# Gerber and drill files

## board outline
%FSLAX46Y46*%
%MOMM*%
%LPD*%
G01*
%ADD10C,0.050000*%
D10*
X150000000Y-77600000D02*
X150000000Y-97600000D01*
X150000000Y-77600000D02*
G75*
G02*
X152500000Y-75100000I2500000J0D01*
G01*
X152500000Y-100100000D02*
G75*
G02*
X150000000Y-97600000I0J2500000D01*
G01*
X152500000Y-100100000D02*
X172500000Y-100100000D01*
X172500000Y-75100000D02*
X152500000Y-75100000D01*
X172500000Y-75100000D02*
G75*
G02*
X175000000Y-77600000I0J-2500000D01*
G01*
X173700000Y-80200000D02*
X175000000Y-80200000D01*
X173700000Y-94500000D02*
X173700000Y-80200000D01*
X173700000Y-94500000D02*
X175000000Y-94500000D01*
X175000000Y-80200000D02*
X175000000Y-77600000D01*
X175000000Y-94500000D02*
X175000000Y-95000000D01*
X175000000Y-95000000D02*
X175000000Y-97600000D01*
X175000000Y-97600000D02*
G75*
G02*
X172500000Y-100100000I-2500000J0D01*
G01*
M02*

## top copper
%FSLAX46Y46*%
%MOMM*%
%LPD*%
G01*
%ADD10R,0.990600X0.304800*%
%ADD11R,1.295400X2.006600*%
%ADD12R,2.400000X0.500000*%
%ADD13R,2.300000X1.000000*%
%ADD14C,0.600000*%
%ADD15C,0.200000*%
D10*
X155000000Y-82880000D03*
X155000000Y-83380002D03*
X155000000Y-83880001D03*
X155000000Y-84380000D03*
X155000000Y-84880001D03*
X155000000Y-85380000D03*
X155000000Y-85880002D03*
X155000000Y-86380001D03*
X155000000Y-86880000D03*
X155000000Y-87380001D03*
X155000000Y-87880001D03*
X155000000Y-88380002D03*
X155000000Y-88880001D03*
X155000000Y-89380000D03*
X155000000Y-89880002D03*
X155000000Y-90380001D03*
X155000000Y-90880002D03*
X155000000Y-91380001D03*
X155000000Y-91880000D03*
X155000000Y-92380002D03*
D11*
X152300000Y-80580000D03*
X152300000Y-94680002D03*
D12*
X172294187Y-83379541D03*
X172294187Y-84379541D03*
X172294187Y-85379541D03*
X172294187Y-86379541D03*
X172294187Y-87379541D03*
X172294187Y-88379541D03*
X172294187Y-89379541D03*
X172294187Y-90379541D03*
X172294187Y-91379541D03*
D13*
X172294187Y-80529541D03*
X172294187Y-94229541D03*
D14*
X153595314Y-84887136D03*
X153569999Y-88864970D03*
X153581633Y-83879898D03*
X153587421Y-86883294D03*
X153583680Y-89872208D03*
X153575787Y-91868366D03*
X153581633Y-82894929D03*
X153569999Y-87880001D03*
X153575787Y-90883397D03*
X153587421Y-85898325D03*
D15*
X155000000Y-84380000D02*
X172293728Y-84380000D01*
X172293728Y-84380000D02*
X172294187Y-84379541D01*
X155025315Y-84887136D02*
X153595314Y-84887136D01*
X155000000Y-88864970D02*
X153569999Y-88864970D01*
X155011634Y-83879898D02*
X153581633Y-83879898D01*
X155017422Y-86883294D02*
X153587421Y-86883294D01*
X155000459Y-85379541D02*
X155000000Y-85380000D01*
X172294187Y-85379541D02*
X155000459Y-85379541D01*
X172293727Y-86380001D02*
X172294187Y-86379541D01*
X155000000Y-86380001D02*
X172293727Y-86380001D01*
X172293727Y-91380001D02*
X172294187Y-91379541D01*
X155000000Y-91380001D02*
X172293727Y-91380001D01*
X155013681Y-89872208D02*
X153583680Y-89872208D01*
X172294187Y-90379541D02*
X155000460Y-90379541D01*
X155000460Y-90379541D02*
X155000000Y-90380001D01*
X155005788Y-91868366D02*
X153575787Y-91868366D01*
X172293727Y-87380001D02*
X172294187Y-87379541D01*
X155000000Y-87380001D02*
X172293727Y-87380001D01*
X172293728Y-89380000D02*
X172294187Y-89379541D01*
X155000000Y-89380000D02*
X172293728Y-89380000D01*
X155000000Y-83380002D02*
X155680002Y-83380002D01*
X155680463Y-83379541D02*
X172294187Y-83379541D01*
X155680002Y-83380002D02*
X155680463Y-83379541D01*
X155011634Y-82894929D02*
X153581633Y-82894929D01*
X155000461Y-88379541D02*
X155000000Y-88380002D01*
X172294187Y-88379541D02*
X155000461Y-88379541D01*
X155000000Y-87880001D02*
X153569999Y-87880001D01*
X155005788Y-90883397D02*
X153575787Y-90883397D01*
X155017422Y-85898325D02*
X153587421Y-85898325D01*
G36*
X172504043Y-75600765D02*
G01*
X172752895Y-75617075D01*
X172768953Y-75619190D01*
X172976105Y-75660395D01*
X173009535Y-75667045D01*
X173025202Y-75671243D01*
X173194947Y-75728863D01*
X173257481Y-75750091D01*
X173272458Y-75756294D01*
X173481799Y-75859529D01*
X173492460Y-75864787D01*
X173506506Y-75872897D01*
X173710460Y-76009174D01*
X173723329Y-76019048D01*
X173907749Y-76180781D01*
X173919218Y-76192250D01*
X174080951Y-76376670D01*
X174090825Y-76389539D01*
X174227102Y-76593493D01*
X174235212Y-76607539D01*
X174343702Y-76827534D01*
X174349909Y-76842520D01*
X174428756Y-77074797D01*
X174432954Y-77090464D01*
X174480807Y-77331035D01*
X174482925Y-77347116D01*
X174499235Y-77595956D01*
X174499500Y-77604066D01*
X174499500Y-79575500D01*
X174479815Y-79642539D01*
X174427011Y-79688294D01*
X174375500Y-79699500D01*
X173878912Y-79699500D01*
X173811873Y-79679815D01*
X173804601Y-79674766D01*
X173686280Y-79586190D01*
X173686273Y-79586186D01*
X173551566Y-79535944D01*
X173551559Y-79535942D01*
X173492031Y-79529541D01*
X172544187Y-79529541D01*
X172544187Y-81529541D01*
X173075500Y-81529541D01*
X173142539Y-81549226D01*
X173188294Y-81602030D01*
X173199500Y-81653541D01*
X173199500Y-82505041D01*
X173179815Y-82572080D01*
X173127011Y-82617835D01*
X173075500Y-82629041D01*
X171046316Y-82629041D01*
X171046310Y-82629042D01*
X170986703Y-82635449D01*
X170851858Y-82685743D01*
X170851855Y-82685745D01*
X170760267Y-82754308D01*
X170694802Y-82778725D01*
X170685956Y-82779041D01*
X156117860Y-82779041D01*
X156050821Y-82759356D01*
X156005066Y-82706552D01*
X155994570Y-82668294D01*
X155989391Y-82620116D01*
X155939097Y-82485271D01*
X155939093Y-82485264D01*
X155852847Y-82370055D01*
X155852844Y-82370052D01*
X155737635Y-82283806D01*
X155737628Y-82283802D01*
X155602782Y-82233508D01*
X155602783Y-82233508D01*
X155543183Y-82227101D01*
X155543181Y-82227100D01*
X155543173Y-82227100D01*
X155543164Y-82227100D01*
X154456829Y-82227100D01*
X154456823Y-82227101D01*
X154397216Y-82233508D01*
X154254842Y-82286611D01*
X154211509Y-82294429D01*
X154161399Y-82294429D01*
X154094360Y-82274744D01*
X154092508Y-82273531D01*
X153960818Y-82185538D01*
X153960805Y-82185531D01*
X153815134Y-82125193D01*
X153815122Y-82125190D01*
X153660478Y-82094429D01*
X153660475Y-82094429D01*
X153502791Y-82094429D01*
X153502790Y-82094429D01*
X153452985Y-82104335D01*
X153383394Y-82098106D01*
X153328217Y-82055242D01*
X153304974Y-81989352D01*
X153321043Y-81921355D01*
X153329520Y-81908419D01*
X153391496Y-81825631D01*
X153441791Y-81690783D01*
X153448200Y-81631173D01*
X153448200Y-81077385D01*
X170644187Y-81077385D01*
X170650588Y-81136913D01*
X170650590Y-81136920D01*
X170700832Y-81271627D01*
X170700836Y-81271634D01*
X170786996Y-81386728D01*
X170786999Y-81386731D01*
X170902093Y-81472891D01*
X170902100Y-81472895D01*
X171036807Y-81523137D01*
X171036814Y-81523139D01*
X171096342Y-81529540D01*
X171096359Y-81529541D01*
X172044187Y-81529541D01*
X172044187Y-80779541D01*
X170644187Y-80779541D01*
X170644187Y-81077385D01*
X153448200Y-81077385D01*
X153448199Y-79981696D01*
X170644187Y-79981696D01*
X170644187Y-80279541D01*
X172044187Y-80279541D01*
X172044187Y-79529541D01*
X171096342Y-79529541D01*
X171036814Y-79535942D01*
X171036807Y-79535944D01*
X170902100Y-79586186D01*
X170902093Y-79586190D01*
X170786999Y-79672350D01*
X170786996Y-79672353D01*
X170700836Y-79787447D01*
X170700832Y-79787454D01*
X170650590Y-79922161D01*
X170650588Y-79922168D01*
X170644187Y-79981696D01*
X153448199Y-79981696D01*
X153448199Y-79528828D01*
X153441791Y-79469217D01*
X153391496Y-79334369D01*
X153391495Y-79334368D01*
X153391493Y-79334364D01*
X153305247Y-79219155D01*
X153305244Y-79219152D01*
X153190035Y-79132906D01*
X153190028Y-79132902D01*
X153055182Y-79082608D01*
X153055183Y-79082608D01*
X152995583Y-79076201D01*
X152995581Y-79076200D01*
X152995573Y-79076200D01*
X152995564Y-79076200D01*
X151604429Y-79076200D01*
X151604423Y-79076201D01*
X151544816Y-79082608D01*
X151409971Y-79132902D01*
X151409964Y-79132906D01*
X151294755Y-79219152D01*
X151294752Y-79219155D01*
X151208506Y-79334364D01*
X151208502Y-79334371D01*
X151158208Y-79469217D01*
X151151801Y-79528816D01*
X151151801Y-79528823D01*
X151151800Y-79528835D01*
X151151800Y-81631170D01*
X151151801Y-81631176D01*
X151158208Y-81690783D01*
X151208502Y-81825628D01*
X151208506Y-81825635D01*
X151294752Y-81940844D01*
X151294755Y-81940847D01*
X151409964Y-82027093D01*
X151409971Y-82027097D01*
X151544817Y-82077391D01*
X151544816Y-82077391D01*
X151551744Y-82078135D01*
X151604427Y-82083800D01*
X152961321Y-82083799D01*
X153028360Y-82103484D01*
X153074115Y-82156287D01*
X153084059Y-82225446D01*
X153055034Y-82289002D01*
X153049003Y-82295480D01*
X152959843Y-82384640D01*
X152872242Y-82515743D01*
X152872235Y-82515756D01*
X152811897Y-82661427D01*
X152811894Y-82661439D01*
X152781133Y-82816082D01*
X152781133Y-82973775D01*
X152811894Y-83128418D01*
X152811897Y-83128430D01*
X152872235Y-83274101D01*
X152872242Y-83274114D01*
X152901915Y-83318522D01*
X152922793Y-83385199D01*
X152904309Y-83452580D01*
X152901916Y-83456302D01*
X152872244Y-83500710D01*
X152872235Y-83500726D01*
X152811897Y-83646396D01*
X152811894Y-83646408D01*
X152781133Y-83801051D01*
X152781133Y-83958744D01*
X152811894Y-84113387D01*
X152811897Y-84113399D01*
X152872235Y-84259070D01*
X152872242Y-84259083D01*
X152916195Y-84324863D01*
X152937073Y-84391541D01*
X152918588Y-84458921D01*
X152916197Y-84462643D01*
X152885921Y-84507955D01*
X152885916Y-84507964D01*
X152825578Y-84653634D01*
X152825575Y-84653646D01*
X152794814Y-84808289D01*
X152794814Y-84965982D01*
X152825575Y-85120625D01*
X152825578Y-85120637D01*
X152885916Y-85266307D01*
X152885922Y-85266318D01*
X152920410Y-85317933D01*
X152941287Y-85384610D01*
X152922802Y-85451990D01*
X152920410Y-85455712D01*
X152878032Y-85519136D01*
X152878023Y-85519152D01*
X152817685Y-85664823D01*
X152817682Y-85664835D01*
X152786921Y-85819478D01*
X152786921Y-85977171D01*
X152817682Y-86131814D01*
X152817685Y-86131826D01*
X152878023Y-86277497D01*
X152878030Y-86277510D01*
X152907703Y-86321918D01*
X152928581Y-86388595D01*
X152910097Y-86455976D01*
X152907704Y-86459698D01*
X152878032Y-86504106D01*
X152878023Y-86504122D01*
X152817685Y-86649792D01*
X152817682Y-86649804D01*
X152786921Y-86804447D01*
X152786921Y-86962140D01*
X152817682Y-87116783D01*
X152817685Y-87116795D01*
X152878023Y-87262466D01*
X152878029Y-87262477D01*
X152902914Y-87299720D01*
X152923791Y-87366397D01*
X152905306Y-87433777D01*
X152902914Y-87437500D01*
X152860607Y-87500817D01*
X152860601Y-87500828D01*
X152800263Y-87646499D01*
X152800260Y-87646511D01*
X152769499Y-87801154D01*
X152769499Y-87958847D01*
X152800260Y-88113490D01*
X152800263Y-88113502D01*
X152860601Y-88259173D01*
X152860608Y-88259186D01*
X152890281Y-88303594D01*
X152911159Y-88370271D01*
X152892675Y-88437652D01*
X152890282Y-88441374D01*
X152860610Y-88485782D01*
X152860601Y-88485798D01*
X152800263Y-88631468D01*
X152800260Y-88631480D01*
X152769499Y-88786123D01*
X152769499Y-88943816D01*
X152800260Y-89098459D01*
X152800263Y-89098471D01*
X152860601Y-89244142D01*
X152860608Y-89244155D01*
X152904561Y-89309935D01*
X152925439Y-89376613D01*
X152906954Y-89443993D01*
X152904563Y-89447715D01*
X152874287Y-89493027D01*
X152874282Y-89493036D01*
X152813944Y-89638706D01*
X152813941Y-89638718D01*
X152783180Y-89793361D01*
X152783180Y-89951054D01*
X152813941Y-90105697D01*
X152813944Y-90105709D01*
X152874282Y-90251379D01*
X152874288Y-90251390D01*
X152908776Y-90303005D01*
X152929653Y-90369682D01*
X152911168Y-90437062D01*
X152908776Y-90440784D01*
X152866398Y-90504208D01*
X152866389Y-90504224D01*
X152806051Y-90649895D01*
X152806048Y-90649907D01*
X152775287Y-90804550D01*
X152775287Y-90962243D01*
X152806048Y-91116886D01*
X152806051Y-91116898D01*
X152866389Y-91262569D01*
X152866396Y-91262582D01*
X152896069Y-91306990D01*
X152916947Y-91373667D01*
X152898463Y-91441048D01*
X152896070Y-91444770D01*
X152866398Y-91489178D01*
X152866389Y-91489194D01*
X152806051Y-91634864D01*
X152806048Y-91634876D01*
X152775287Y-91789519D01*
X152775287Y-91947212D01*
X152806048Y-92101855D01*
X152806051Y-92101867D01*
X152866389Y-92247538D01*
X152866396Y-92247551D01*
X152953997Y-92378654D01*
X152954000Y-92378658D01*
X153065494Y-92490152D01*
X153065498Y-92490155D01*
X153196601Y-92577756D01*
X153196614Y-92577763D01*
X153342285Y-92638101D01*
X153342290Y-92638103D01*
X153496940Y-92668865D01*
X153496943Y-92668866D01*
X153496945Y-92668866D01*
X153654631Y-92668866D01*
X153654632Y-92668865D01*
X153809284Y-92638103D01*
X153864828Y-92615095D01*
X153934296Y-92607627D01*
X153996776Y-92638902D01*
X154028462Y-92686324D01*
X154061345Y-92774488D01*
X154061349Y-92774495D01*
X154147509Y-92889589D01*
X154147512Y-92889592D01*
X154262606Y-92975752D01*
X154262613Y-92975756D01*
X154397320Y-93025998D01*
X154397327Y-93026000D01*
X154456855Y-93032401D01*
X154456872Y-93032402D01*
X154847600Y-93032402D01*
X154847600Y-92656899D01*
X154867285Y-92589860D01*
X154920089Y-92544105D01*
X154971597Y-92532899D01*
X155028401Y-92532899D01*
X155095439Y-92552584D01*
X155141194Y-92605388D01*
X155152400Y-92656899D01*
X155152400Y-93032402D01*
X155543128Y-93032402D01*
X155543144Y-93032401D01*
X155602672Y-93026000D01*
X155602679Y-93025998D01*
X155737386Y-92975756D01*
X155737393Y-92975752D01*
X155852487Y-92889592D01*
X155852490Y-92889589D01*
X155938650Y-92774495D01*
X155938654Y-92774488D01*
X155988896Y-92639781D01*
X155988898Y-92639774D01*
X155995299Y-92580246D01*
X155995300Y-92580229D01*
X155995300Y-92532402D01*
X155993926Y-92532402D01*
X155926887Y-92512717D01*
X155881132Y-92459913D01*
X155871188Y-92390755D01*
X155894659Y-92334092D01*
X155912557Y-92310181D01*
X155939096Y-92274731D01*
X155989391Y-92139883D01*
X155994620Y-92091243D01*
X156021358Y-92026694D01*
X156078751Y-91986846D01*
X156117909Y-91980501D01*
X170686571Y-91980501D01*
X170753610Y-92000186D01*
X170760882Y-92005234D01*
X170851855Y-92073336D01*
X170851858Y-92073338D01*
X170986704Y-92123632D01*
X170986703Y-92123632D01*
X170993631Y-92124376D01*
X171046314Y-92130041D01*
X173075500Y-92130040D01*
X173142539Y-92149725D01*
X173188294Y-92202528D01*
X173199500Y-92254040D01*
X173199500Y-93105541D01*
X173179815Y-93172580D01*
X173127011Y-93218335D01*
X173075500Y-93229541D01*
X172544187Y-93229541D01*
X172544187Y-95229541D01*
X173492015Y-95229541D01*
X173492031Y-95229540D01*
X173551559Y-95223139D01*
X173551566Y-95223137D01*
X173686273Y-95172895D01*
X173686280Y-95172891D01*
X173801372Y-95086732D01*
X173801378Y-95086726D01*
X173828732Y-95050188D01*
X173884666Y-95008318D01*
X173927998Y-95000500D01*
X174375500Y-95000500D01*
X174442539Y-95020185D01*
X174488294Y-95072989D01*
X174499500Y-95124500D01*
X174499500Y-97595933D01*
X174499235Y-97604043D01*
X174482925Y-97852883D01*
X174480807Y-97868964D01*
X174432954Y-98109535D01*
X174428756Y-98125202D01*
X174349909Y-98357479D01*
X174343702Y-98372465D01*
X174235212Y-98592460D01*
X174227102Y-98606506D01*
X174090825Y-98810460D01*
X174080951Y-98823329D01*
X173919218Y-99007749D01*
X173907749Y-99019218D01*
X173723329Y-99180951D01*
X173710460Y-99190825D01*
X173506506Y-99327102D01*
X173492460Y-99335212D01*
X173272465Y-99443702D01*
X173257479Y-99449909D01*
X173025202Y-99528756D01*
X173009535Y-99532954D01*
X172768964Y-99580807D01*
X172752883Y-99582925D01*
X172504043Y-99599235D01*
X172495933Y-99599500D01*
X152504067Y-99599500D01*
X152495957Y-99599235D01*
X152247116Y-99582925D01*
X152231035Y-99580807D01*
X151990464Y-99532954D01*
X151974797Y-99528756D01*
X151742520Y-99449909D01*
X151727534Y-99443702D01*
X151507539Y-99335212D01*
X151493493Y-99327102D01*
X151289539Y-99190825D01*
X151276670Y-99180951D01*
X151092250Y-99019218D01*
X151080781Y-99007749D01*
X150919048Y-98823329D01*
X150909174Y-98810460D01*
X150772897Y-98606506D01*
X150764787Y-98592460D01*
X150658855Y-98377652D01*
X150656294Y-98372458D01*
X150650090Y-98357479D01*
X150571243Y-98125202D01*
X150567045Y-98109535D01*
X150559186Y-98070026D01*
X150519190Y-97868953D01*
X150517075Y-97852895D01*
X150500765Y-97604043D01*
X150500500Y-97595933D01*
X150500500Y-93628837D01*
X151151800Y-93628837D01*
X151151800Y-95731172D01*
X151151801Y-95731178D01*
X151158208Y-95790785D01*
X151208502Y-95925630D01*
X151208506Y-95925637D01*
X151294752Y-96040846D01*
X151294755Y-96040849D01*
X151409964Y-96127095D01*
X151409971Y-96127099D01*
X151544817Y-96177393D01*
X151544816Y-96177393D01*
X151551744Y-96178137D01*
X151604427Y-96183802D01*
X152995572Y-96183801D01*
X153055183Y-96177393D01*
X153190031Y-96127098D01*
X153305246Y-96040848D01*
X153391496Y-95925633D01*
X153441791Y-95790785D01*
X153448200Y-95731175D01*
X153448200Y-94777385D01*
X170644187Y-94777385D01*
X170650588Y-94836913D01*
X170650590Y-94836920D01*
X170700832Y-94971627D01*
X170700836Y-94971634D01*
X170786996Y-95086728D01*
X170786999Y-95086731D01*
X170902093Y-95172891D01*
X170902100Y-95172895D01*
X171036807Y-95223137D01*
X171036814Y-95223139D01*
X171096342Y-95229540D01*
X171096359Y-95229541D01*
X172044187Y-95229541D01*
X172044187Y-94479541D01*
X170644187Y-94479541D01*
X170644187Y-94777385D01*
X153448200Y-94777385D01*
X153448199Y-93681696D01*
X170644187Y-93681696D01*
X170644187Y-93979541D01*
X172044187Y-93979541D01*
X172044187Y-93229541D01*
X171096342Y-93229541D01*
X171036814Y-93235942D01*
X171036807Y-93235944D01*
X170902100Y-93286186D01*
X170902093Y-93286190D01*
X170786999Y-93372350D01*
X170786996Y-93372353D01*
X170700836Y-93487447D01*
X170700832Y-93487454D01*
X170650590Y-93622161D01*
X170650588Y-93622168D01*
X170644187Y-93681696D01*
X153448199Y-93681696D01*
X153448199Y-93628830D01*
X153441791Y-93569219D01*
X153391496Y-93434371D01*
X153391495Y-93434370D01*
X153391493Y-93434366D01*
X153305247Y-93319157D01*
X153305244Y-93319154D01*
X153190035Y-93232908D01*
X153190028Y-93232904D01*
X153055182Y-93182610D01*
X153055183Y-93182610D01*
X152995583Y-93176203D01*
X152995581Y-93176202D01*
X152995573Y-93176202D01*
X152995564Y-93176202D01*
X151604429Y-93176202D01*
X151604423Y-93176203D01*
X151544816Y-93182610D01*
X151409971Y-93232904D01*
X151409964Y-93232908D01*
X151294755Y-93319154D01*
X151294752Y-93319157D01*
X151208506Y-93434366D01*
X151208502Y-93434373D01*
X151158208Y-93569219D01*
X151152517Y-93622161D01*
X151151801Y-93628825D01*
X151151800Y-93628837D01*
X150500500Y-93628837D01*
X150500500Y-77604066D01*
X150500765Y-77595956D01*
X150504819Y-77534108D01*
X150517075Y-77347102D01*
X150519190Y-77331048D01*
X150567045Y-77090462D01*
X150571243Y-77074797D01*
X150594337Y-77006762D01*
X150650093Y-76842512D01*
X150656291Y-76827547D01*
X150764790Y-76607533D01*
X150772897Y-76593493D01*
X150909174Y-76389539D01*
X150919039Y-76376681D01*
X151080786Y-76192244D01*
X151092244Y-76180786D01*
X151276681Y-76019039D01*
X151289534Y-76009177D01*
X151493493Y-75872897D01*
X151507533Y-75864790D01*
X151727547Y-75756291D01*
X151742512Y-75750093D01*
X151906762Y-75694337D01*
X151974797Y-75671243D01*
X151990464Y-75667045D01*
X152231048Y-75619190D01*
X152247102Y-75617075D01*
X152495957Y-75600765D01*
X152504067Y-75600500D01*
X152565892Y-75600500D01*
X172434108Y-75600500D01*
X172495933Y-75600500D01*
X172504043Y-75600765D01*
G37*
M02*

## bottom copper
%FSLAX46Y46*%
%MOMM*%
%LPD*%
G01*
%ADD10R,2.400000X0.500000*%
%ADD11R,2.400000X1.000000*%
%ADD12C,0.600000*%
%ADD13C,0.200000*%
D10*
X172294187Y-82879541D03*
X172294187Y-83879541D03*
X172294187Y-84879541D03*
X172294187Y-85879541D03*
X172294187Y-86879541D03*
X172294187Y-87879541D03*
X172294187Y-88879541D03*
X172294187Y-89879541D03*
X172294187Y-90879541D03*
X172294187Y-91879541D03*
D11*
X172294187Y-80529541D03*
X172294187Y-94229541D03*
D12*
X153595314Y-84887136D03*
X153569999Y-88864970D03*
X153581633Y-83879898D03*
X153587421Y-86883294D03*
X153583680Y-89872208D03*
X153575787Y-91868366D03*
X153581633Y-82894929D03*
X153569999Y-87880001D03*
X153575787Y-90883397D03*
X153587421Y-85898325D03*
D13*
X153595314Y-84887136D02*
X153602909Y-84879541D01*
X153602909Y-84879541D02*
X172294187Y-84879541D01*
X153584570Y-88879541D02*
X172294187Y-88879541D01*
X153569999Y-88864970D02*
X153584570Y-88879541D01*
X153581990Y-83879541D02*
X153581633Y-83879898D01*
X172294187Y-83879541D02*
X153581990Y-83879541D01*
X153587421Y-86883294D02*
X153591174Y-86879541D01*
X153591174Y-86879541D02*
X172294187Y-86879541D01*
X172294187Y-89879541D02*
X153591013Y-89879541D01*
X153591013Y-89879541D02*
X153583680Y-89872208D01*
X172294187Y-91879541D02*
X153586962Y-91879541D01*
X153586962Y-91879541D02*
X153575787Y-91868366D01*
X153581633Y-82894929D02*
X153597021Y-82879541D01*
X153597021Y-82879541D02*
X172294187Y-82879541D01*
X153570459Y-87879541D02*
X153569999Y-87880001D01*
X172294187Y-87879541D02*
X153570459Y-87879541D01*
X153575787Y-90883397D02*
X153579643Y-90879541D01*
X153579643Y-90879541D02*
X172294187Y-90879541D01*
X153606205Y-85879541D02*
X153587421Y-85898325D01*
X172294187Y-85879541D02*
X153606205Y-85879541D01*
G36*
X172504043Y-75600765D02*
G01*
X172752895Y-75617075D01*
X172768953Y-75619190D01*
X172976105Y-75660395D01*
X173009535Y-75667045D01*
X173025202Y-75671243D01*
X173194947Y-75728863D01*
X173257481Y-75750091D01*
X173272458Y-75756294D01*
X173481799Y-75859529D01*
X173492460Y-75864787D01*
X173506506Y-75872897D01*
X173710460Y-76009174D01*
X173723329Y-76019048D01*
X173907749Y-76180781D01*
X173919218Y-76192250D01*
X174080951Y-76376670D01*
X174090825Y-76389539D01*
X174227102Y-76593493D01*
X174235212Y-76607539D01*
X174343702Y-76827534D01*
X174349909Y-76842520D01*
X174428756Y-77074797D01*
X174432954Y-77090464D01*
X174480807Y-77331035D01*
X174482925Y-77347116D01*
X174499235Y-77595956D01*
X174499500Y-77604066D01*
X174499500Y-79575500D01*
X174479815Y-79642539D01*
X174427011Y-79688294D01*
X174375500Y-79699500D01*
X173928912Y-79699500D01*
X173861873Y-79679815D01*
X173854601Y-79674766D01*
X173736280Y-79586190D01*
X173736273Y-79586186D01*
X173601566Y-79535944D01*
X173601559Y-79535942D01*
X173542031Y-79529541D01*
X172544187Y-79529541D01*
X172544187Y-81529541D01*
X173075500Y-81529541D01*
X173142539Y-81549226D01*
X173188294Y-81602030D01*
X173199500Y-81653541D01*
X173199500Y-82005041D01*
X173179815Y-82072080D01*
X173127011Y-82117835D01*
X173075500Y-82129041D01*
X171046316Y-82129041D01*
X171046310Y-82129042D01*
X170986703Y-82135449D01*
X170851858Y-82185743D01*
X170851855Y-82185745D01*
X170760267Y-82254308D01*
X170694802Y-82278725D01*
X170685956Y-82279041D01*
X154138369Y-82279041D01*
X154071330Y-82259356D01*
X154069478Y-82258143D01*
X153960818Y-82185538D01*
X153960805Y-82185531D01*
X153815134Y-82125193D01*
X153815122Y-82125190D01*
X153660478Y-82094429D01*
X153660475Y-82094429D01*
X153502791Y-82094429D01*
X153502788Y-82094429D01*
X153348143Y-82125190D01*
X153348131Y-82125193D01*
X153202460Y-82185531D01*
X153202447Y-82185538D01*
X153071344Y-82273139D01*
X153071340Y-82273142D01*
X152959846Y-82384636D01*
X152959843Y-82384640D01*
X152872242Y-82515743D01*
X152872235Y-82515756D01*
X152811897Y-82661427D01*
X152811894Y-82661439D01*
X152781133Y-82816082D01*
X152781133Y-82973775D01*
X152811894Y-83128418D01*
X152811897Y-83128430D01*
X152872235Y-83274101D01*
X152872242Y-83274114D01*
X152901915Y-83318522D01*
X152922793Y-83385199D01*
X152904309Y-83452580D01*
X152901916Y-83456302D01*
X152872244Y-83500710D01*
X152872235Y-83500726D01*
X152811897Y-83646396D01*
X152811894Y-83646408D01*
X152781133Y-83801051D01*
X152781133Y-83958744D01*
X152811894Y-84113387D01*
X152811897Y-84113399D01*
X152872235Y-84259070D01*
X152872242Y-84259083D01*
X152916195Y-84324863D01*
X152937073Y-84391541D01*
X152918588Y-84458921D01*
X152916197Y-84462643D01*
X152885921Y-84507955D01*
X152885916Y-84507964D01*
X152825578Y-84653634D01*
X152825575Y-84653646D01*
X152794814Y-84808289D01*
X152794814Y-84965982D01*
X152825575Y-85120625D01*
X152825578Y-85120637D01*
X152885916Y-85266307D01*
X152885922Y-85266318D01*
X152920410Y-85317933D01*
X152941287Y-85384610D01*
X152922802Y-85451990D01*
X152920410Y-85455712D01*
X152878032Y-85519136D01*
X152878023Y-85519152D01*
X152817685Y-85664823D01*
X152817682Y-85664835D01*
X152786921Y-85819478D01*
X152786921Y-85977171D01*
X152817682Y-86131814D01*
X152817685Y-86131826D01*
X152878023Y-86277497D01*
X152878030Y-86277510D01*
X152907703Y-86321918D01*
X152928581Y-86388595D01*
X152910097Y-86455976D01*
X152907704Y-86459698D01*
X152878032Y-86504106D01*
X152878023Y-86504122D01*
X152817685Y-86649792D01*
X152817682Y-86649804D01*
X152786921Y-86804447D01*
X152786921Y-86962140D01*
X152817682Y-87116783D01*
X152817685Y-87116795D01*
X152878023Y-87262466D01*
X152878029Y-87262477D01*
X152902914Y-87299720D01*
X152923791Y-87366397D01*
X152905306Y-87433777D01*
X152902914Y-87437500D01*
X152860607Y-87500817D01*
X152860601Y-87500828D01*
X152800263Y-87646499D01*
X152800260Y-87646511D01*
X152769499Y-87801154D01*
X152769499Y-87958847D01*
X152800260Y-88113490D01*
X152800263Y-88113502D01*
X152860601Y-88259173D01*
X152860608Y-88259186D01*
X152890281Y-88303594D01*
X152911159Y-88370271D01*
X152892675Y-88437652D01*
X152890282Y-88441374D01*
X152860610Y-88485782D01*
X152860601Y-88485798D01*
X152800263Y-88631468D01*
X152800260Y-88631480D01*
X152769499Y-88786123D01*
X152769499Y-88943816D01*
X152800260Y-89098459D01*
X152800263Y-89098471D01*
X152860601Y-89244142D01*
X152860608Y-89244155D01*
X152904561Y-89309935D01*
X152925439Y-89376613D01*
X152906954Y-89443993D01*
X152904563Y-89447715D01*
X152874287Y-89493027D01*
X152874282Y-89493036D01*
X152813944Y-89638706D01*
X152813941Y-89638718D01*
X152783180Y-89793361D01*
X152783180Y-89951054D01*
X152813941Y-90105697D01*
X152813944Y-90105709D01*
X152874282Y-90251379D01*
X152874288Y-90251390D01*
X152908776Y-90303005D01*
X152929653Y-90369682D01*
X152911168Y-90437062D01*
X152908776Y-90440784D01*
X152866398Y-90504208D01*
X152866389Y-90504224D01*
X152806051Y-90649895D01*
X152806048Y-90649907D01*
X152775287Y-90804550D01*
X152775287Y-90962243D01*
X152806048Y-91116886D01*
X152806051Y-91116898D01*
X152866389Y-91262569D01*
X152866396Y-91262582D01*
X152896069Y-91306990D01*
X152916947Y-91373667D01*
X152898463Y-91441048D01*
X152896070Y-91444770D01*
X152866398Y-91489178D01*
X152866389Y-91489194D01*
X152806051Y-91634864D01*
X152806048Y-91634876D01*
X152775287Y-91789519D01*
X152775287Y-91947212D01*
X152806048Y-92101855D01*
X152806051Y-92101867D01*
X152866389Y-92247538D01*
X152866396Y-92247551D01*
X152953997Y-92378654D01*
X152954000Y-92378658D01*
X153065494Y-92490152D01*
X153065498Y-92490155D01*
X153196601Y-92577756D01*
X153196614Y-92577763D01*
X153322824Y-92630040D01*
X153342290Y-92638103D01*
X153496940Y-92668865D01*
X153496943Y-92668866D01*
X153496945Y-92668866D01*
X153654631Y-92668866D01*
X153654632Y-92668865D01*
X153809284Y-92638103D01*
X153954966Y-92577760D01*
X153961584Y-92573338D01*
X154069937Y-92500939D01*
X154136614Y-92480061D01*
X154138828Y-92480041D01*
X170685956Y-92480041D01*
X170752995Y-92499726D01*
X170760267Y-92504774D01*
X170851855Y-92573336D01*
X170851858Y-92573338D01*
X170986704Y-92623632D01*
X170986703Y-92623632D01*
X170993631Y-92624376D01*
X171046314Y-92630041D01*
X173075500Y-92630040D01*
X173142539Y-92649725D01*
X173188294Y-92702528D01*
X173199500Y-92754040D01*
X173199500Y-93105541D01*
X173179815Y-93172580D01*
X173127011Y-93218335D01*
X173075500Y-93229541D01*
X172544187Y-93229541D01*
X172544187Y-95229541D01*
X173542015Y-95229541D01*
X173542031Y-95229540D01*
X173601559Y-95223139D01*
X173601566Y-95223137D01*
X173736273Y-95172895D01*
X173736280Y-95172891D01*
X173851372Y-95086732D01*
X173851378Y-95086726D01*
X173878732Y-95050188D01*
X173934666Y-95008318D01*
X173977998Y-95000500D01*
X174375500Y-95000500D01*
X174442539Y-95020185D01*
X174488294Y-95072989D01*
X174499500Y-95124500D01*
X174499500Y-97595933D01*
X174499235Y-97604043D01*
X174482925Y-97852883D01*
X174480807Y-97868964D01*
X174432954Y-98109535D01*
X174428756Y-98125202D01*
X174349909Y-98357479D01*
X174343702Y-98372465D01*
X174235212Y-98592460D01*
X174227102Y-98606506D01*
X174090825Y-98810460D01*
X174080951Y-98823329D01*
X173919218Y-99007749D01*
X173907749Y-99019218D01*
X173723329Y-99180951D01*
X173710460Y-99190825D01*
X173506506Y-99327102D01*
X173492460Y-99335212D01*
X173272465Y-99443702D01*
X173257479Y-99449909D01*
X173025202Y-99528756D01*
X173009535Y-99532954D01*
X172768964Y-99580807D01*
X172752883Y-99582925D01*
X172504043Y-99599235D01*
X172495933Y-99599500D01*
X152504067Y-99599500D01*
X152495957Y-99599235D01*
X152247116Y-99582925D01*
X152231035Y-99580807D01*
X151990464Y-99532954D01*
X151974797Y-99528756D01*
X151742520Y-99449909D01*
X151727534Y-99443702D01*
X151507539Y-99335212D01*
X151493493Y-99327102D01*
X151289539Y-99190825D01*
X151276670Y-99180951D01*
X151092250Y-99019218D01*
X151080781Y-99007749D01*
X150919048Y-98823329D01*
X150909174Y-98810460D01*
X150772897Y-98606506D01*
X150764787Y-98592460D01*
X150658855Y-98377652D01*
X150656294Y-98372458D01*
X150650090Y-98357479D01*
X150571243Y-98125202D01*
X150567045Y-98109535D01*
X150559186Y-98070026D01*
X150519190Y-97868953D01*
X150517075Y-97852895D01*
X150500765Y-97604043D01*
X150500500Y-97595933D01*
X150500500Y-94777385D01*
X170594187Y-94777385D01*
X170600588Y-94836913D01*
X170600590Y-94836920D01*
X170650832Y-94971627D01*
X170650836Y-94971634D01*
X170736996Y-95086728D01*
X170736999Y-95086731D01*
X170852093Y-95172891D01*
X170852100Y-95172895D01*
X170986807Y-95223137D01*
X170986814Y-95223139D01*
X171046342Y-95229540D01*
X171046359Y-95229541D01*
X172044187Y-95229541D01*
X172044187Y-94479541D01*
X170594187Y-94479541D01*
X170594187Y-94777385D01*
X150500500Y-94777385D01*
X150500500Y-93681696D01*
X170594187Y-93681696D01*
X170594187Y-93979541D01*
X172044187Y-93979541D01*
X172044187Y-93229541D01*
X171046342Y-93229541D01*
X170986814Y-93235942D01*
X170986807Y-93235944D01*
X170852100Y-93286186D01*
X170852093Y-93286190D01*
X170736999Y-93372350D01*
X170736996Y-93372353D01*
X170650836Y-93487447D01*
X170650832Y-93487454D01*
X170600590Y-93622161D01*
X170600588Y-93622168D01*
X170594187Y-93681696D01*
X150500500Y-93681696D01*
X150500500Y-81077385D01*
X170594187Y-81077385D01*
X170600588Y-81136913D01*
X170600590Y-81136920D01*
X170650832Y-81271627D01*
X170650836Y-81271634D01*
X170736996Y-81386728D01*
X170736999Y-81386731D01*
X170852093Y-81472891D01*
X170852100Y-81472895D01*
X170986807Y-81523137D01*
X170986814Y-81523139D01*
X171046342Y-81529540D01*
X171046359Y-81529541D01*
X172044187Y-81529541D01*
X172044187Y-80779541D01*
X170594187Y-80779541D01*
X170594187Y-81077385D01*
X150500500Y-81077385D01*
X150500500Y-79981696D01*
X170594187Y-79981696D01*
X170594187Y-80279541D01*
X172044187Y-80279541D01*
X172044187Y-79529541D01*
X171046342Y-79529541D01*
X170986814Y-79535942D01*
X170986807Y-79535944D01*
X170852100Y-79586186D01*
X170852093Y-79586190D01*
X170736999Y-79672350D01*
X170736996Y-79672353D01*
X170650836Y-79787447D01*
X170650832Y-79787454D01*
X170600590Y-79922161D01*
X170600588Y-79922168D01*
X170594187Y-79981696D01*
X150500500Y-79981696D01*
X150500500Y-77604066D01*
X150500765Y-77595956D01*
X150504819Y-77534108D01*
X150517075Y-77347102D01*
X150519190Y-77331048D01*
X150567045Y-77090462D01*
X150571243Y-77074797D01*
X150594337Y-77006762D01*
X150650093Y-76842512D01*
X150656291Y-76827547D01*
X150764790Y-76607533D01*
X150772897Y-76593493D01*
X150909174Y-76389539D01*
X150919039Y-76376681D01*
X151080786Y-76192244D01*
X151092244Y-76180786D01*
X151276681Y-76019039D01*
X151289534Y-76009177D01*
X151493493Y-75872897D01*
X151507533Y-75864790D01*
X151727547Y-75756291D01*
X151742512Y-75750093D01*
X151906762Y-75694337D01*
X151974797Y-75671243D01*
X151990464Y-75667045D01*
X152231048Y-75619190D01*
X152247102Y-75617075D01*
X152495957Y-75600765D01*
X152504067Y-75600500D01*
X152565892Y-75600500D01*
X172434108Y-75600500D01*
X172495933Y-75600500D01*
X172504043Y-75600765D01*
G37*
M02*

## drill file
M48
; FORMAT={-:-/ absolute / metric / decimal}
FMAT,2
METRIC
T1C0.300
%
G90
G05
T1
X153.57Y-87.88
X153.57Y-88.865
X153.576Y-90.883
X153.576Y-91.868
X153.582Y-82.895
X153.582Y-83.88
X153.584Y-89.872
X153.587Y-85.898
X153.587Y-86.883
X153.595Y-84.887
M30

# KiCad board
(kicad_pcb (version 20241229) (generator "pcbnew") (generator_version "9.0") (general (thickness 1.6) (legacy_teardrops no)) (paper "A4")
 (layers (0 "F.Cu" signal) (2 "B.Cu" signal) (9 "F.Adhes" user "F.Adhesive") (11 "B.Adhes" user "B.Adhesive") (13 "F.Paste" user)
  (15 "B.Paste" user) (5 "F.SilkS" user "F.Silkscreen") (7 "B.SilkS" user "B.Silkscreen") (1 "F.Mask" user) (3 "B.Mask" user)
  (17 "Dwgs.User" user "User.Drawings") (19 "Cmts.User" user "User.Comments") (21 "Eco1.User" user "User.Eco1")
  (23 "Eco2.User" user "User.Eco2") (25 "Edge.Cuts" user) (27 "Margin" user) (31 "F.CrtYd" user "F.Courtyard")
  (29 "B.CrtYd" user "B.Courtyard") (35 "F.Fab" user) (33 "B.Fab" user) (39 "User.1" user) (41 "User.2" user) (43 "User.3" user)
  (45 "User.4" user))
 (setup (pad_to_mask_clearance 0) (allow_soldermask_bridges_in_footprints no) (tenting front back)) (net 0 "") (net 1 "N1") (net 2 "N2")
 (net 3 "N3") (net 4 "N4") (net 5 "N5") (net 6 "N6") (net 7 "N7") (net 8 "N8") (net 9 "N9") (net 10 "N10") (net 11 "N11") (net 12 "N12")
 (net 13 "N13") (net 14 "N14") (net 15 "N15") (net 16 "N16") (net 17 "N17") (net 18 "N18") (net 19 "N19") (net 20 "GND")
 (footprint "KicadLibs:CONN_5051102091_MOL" (layer "F.Cu") (at 152.5211 87.630001 -90)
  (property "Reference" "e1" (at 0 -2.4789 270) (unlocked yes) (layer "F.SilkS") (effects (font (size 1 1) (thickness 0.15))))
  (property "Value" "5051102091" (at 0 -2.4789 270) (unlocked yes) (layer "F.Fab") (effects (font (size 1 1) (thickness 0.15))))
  (pad "1" smd rect (at -4.750001 -2.4789 270) (size 0.3048 0.9906) (layers "F.Cu" "F.Mask" "F.Paste") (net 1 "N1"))
  (pad "2" smd rect (at -4.249999 -2.4789 270) (size 0.3048 0.9906) (layers "F.Cu" "F.Mask" "F.Paste") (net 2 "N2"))
  (pad "3" smd rect (at -3.75 -2.4789 270) (size 0.3048 0.9906) (layers "F.Cu" "F.Mask" "F.Paste") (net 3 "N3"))
  (pad "4" smd rect (at -3.250001 -2.4789 270) (size 0.3048 0.9906) (layers "F.Cu" "F.Mask" "F.Paste") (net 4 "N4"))
  (pad "5" smd rect (at -2.75 -2.4789 270) (size 0.3048 0.9906) (layers "F.Cu" "F.Mask" "F.Paste") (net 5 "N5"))
  (pad "6" smd rect (at -2.250001 -2.4789 270) (size 0.3048 0.9906) (layers "F.Cu" "F.Mask" "F.Paste") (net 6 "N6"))
  (pad "7" smd rect (at -1.749999 -2.4789 270) (size 0.3048 0.9906) (layers "F.Cu" "F.Mask" "F.Paste") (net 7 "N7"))
  (pad "8" smd rect (at -1.25 -2.4789 270) (size 0.3048 0.9906) (layers "F.Cu" "F.Mask" "F.Paste") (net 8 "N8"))
  (pad "9" smd rect (at -0.750001 -2.4789 270) (size 0.3048 0.9906) (layers "F.Cu" "F.Mask" "F.Paste") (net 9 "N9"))
  (pad "10" smd rect (at -0.25 -2.4789 270) (size 0.3048 0.9906) (layers "F.Cu" "F.Mask" "F.Paste") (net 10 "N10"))
  (pad "11" smd rect (at 0.25 -2.4789 270) (size 0.3048 0.9906) (layers "F.Cu" "F.Mask" "F.Paste") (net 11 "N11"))
  (pad "12" smd rect (at 0.750001 -2.4789 270) (size 0.3048 0.9906) (layers "F.Cu" "F.Mask" "F.Paste") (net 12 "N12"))
  (pad "13" smd rect (at 1.25 -2.4789 270) (size 0.3048 0.9906) (layers "F.Cu" "F.Mask" "F.Paste") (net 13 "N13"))
  (pad "14" smd rect (at 1.749999 -2.4789 270) (size 0.3048 0.9906) (layers "F.Cu" "F.Mask" "F.Paste") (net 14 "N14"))
  (pad "15" smd rect (at 2.250001 -2.4789 270) (size 0.3048 0.9906) (layers "F.Cu" "F.Mask" "F.Paste") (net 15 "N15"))
  (pad "16" smd rect (at 2.75 -2.4789 270) (size 0.3048 0.9906) (layers "F.Cu" "F.Mask" "F.Paste") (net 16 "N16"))
  (pad "17" smd rect (at 3.250001 -2.4789 270) (size 0.3048 0.9906) (layers "F.Cu" "F.Mask" "F.Paste") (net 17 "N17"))
  (pad "18" smd rect (at 3.75 -2.4789 270) (size 0.3048 0.9906) (layers "F.Cu" "F.Mask" "F.Paste") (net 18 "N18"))
  (pad "19" smd rect (at 4.249999 -2.4789 270) (size 0.3048 0.9906) (layers "F.Cu" "F.Mask" "F.Paste") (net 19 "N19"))
  (pad "20" smd rect (at 4.750001 -2.4789 270) (size 0.3048 0.9906) (layers "F.Cu" "F.Mask" "F.Paste") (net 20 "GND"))
  (pad "21" smd rect (at -7.050001 0.2211 270) (size 2.0066 1.2954) (layers "F.Cu" "F.Mask" "F.Paste"))
  (pad "22" smd rect (at 7.050001 0.2211 270) (size 2.0066 1.2954) (layers "F.Cu" "F.Mask" "F.Paste")))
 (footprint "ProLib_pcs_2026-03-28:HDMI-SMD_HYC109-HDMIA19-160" (layer "B.Cu") (at 172.294187 87.379541 -90)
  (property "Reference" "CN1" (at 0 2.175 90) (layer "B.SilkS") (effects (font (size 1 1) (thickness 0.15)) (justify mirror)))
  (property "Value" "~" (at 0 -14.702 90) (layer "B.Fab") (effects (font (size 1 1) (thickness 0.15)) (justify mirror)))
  (pad "1" smd rect (at -4.5 0 270) (size 0.5 2.4) (layers "B.Cu" "B.Mask" "B.Paste") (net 1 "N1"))
  (pad "2" smd rect (at -4 0 270) (size 0.5 2.4) (layers "F.Cu" "F.Mask" "F.Paste") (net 2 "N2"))
  (pad "3" smd rect (at -3.5 0 270) (size 0.5 2.4) (layers "B.Cu" "B.Mask" "B.Paste") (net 3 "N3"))
  (pad "4" smd rect (at -3 0 270) (size 0.5 2.4) (layers "F.Cu" "F.Mask" "F.Paste") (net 4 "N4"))
  (pad "5" smd rect (at -2.5 0 270) (size 0.5 2.4) (layers "B.Cu" "B.Mask" "B.Paste") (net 5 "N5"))
  (pad "6" smd rect (at -2 0 270) (size 0.5 2.4) (layers "F.Cu" "F.Mask" "F.Paste") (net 6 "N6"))
  (pad "7" smd rect (at -1.5 0 270) (size 0.5 2.4) (layers "B.Cu" "B.Mask" "B.Paste") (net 7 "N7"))
  (pad "8" smd rect (at -1 0 270) (size 0.5 2.4) (layers "F.Cu" "F.Mask" "F.Paste") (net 8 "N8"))
  (pad "9" smd rect (at -0.5 0 270) (size 0.5 2.4) (layers "B.Cu" "B.Mask" "B.Paste") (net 9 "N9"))
  (pad "10" smd rect (at 0 0 270) (size 0.5 2.4) (layers "F.Cu" "F.Mask" "F.Paste") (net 10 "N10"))
  (pad "11" smd rect (at 0.5 0 270) (size 0.5 2.4) (layers "B.Cu" "B.Mask" "B.Paste") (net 11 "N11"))
  (pad "12" smd rect (at 1 0 270) (size 0.5 2.4) (layers "F.Cu" "F.Mask" "F.Paste") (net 12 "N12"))
  (pad "13" smd rect (at 1.5 0 270) (size 0.5 2.4) (layers "B.Cu" "B.Mask" "B.Paste") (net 13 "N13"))
  (pad "14" smd rect (at 2 0 270) (size 0.5 2.4) (layers "F.Cu" "F.Mask" "F.Paste") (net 14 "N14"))
  (pad "15" smd rect (at 2.5 0 270) (size 0.5 2.4) (layers "B.Cu" "B.Mask" "B.Paste") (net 15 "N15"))
  (pad "16" smd rect (at 3 0 270) (size 0.5 2.4) (layers "F.Cu" "F.Mask" "F.Paste") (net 16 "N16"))
  (pad "17" smd rect (at 3.5 0 270) (size 0.5 2.4) (layers "B.Cu" "B.Mask" "B.Paste") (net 17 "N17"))
  (pad "18" smd rect (at 4 0 270) (size 0.5 2.4) (layers "F.Cu" "F.Mask" "F.Paste") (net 18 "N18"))
  (pad "19" smd rect (at 4.5 0 270) (size 0.5 2.4) (layers "B.Cu" "B.Mask" "B.Paste") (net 19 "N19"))
  (pad "20" smd rect (at -6.85 0 270) (size 1 2.4) (layers "B.Cu" "B.Mask" "B.Paste") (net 20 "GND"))
  (pad "21" smd rect (at 6.85 0 270) (size 1 2.4) (layers "B.Cu" "B.Mask" "B.Paste") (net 20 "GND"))
  (pad "22" smd rect (at -6.85 0 270) (size 1 2.3) (layers "F.Cu" "F.Mask" "F.Paste") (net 20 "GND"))
  (pad "23" smd rect (at 6.85 0 270) (size 1 2.3) (layers "F.Cu" "F.Mask" "F.Paste") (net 20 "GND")))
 (gr_line (start 150 77.6) (end 150 97.6) (stroke (width 0.05) (type default)) (layer "Edge.Cuts"))
 (gr_arc (start 150 77.6) (mid 150.732233 75.832233) (end 152.5 75.1) (stroke (width 0.05) (type default)) (layer "Edge.Cuts"))
 (gr_arc (start 152.5 100.1) (mid 150.732233 99.367767) (end 150 97.6) (stroke (width 0.05) (type default)) (layer "Edge.Cuts"))
 (gr_line (start 152.5 100.1) (end 172.5 100.1) (stroke (width 0.05) (type default)) (layer "Edge.Cuts"))
 (gr_line (start 172.5 75.1) (end 152.5 75.1) (stroke (width 0.05) (type default)) (layer "Edge.Cuts"))
 (gr_arc (start 172.5 75.1) (mid 174.267767 75.832233) (end 175 77.6) (stroke (width 0.05) (type default)) (layer "Edge.Cuts"))
 (gr_line (start 173.7 80.2) (end 175 80.2) (stroke (width 0.05) (type solid)) (layer "Edge.Cuts"))
 (gr_line (start 173.7 94.5) (end 173.7 80.2) (stroke (width 0.05) (type default)) (layer "Edge.Cuts"))
 (gr_line (start 173.7 94.5) (end 175 94.5) (stroke (width 0.05) (type default)) (layer "Edge.Cuts"))
 (gr_line (start 175 80.2) (end 175 77.6) (stroke (width 0.05) (type default)) (layer "Edge.Cuts"))
 (gr_line (start 175 94.5) (end 175 95) (stroke (width 0.05) (type default)) (layer "Edge.Cuts"))
 (gr_line (start 175 95) (end 175 97.6) (stroke (width 0.05) (type default)) (layer "Edge.Cuts"))
 (gr_arc (start 175 97.6) (mid 174.267767 99.367767) (end 172.5 100.1) (stroke (width 0.05) (type default)) (layer "Edge.Cuts"))
 (segment (start 155 84.38) (end 172.293728 84.38) (width 0.2) (layer "F.Cu") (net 4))
 (segment (start 172.293728 84.38) (end 172.294187 84.379541) (width 0.2) (layer "F.Cu") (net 4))
 (segment (start 155.025315 84.887136) (end 153.595314 84.887136) (width 0.2) (layer "F.Cu") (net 5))
 (via (at 153.595314 84.887136) (size 0.6) (drill 0.3) (layers "F.Cu" "B.Cu") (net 5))
 (segment (start 153.595314 84.887136) (end 153.602909 84.879541) (width 0.2) (layer "B.Cu") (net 5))
 (segment (start 153.602909 84.879541) (end 172.294187 84.879541) (width 0.2) (layer "B.Cu") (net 5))
 (segment (start 155 88.86497) (end 153.569999 88.86497) (width 0.2) (layer "F.Cu") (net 13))
 (via (at 153.569999 88.86497) (size 0.6) (drill 0.3) (layers "F.Cu" "B.Cu") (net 13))
 (segment (start 153.58457 88.879541) (end 172.294187 88.879541) (width 0.2) (layer "B.Cu") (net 13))
 (segment (start 153.569999 88.86497) (end 153.58457 88.879541) (width 0.2) (layer "B.Cu") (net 13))
 (segment (start 155.011634 83.879898) (end 153.581633 83.879898) (width 0.2) (layer "F.Cu") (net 3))
 (via (at 153.581633 83.879898) (size 0.6) (drill 0.3) (layers "F.Cu" "B.Cu") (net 3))
 (segment (start 153.58199 83.879541) (end 153.581633 83.879898) (width 0.2) (layer "B.Cu") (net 3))
 (segment (start 172.294187 83.879541) (end 153.58199 83.879541) (width 0.2) (layer "B.Cu") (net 3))
 (segment (start 155.017422 86.883294) (end 153.587421 86.883294) (width 0.2) (layer "F.Cu") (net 9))
 (via (at 153.587421 86.883294) (size 0.6) (drill 0.3) (layers "F.Cu" "B.Cu") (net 9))
 (segment (start 153.587421 86.883294) (end 153.591174 86.879541) (width 0.2) (layer "B.Cu") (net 9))
 (segment (start 153.591174 86.879541) (end 172.294187 86.879541) (width 0.2) (layer "B.Cu") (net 9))
 (segment (start 155.000459 85.379541) (end 155 85.38) (width 0.2) (layer "F.Cu") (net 6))
 (segment (start 172.294187 85.379541) (end 155.000459 85.379541) (width 0.2) (layer "F.Cu") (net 6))
 (segment (start 172.293727 86.380001) (end 172.294187 86.379541) (width 0.2) (layer "F.Cu") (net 8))
 (segment (start 155 86.380001) (end 172.293727 86.380001) (width 0.2) (layer "F.Cu") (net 8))
 (segment (start 172.293727 91.380001) (end 172.294187 91.379541) (width 0.2) (layer "F.Cu") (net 18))
 (segment (start 155 91.380001) (end 172.293727 91.380001) (width 0.2) (layer "F.Cu") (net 18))
 (segment (start 155.013681 89.872208) (end 153.58368 89.872208) (width 0.2) (layer "F.Cu") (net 15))
 (via (at 153.58368 89.872208) (size 0.6) (drill 0.3) (layers "F.Cu" "B.Cu") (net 15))
 (segment (start 172.294187 89.879541) (end 153.591013 89.879541) (width 0.2) (layer "B.Cu") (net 15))
 (segment (start 153.591013 89.879541) (end 153.58368 89.872208) (width 0.2) (layer "B.Cu") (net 15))
 (segment (start 172.294187 90.379541) (end 155.00046 90.379541) (width 0.2) (layer "F.Cu") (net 16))
 (segment (start 155.00046 90.379541) (end 155 90.380001) (width 0.2) (layer "F.Cu") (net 16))
 (segment (start 155.005788 91.868366) (end 153.575787 91.868366) (width 0.2) (layer "F.Cu") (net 19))
 (via (at 153.575787 91.868366) (size 0.6) (drill 0.3) (layers "F.Cu" "B.Cu") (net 19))
 (segment (start 172.294187 91.879541) (end 153.586962 91.879541) (width 0.2) (layer "B.Cu") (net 19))
 (segment (start 153.586962 91.879541) (end 153.575787 91.868366) (width 0.2) (layer "B.Cu") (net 19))
 (segment (start 172.293727 87.380001) (end 172.294187 87.379541) (width 0.2) (layer "F.Cu") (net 10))
 (segment (start 155 87.380001) (end 172.293727 87.380001) (width 0.2) (layer "F.Cu") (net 10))
 (segment (start 172.293728 89.38) (end 172.294187 89.379541) (width 0.2) (layer "F.Cu") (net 14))
 (segment (start 155 89.38) (end 172.293728 89.38) (width 0.2) (layer "F.Cu") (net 14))
 (segment (start 155 83.380002) (end 155.680002 83.380002) (width 0.2) (layer "F.Cu") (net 2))
 (segment (start 155.680463 83.379541) (end 172.294187 83.379541) (width 0.2) (layer "F.Cu") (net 2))
 (segment (start 155.680002 83.380002) (end 155.680463 83.379541) (width 0.2) (layer "F.Cu") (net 2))
 (segment (start 155.011634 82.894929) (end 153.581633 82.894929) (width 0.2) (layer "F.Cu") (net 1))
 (via (at 153.581633 82.894929) (size 0.6) (drill 0.3) (layers "F.Cu" "B.Cu") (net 1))
 (segment (start 153.581633 82.894929) (end 153.597021 82.879541) (width 0.2) (layer "B.Cu") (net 1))
 (segment (start 153.597021 82.879541) (end 172.294187 82.879541) (width 0.2) (layer "B.Cu") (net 1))
 (segment (start 155.000461 88.379541) (end 155 88.380002) (width 0.2) (layer "F.Cu") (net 12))
 (segment (start 172.294187 88.379541) (end 155.000461 88.379541) (width 0.2) (layer "F.Cu") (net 12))
 (segment (start 155 87.880001) (end 153.569999 87.880001) (width 0.2) (layer "F.Cu") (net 11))
 (via (at 153.569999 87.880001) (size 0.6) (drill 0.3) (layers "F.Cu" "B.Cu") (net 11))
 (segment (start 153.570459 87.879541) (end 153.569999 87.880001) (width 0.2) (layer "B.Cu") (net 11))
 (segment (start 172.294187 87.879541) (end 153.570459 87.879541) (width 0.2) (layer "B.Cu") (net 11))
 (segment (start 155.005788 90.883397) (end 153.575787 90.883397) (width 0.2) (layer "F.Cu") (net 17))
 (via (at 153.575787 90.883397) (size 0.6) (drill 0.3) (layers "F.Cu" "B.Cu") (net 17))
 (segment (start 153.575787 90.883397) (end 153.579643 90.879541) (width 0.2) (layer "B.Cu") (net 17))
 (segment (start 153.579643 90.879541) (end 172.294187 90.879541) (width 0.2) (layer "B.Cu") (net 17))
 (segment (start 155.017422 85.898325) (end 153.587421 85.898325) (width 0.2) (layer "F.Cu") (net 7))
 (via (at 153.587421 85.898325) (size 0.6) (drill 0.3) (layers "F.Cu" "B.Cu") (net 7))
 (segment (start 153.606205 85.879541) (end 153.587421 85.898325) (width 0.2) (layer "B.Cu") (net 7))
 (segment (start 172.294187 85.879541) (end 153.606205 85.879541) (width 0.2) (layer "B.Cu") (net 7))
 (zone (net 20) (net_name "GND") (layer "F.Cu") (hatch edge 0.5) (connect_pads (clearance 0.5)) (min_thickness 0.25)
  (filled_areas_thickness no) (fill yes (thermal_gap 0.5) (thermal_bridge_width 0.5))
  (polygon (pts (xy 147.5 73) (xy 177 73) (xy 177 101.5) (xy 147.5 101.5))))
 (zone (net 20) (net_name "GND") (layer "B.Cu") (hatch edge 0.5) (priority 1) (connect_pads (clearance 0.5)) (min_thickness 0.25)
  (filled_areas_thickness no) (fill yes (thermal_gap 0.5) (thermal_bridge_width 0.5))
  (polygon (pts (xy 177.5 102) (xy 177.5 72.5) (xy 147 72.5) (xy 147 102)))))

